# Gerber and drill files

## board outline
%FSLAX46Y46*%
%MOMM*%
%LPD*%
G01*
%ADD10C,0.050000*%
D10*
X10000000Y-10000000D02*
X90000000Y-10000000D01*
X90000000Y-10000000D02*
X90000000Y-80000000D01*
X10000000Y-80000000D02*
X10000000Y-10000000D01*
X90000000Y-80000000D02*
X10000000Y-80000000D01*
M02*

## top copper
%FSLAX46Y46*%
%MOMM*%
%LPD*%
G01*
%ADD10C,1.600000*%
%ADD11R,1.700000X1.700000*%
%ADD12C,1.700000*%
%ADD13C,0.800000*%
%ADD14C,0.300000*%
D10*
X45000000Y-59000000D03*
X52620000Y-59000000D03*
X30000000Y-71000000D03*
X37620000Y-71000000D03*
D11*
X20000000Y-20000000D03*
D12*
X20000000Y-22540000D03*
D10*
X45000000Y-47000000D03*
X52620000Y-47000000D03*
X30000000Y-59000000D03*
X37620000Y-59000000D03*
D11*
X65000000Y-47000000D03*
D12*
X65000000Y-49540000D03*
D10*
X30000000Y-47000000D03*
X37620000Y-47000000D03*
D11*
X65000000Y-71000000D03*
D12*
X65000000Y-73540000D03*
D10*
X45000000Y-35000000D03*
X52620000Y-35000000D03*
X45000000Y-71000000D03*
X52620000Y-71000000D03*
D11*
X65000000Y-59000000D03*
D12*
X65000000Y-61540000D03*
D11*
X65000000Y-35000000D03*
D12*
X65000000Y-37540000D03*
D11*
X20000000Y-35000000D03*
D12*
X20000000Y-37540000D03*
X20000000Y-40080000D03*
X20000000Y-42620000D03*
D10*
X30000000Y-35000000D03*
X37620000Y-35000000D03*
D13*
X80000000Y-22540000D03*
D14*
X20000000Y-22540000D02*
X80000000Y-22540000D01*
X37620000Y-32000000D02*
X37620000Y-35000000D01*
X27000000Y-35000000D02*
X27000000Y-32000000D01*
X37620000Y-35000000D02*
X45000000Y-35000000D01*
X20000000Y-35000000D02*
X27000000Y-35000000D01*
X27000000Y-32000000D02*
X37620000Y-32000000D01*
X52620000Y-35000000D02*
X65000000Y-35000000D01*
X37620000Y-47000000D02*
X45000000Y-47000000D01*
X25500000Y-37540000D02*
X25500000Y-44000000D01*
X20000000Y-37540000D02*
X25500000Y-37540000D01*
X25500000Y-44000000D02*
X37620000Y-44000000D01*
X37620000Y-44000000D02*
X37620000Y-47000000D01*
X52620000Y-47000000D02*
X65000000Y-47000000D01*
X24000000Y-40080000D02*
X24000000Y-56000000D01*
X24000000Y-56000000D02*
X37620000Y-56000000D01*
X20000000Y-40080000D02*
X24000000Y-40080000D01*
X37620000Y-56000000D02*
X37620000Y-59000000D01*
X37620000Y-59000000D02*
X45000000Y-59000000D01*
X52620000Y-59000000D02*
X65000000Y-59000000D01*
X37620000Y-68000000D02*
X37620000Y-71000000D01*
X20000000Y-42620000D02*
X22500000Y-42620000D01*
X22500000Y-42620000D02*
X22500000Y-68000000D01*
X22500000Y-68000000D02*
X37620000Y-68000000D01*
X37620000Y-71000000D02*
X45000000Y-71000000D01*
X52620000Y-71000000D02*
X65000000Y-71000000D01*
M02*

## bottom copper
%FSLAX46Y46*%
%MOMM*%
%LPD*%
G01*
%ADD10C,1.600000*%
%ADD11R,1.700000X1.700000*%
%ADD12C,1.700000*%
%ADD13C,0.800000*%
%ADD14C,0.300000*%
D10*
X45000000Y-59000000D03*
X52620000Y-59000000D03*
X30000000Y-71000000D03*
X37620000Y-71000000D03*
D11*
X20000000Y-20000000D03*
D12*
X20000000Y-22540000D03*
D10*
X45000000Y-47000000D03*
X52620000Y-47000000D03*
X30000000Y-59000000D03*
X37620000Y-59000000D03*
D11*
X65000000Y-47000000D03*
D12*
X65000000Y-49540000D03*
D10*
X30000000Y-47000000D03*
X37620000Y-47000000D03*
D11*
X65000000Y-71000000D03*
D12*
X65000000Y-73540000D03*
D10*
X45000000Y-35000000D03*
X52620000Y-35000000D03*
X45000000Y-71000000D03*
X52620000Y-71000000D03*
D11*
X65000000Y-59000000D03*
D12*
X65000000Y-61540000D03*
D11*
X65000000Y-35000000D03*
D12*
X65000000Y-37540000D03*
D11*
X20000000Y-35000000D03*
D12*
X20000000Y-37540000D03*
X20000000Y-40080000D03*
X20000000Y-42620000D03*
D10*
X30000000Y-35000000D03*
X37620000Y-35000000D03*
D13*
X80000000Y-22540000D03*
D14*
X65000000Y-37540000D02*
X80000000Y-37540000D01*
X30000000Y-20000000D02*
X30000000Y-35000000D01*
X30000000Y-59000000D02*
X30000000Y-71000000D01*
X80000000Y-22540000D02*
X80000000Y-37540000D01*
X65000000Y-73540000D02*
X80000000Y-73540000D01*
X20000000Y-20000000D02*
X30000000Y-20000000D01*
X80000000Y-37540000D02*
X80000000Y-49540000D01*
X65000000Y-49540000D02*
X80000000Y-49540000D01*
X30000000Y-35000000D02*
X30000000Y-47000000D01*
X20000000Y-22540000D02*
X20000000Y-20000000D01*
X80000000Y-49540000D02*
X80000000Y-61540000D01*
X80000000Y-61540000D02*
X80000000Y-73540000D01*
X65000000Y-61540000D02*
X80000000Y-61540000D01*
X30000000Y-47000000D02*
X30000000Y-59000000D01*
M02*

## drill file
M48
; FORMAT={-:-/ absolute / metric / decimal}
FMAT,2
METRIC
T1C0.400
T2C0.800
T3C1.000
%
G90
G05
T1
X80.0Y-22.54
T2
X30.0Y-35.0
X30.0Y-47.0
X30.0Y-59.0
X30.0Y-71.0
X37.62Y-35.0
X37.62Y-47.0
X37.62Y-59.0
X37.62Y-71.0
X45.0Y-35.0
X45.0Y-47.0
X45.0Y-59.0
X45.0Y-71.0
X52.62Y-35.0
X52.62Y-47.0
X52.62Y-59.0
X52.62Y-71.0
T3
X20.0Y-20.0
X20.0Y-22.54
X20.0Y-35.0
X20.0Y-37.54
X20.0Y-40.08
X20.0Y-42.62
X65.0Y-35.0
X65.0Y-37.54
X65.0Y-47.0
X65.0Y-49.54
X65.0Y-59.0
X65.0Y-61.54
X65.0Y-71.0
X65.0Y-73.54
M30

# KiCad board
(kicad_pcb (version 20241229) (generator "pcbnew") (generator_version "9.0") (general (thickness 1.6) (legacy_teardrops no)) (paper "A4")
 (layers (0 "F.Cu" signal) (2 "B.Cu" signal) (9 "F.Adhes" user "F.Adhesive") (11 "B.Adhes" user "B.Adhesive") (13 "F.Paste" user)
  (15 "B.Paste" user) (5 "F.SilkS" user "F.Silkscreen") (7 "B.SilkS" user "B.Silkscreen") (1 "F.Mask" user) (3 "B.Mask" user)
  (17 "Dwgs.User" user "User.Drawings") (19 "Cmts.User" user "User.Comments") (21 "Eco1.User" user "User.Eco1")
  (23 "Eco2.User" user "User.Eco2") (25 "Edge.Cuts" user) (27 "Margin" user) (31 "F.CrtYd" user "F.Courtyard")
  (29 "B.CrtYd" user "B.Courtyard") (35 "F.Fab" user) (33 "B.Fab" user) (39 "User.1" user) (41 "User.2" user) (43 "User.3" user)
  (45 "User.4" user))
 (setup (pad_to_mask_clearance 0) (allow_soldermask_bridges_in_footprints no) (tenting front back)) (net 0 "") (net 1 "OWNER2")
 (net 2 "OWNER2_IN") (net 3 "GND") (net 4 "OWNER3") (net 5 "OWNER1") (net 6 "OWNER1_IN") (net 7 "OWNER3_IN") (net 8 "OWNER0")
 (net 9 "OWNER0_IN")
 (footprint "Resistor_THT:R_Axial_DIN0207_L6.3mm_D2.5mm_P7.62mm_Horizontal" (layer "F.Cu") (at 45 59)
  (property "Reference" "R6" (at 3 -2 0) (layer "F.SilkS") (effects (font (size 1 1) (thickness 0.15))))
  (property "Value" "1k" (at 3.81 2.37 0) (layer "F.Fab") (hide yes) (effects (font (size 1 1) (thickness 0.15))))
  (pad "1" thru_hole circle (at 0 0) (size 1.6 1.6) (drill 0.8) (layers "*.Cu" "*.Mask") (remove_unused_layers no) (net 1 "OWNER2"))
  (pad "2" thru_hole circle (at 7.62 0) (size 1.6 1.6) (drill 0.8) (layers "*.Cu" "*.Mask") (remove_unused_layers no) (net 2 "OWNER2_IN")))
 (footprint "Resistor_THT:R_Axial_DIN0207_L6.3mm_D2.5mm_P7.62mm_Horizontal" (layer "F.Cu") (at 30 71)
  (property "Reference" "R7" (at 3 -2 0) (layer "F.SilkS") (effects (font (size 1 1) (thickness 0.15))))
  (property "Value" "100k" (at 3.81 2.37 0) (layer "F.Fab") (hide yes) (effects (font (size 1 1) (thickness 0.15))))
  (pad "1" thru_hole circle (at 0 0) (size 1.6 1.6) (drill 0.8) (layers "*.Cu" "*.Mask") (remove_unused_layers no) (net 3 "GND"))
  (pad "2" thru_hole circle (at 7.62 0) (size 1.6 1.6) (drill 0.8) (layers "*.Cu" "*.Mask") (remove_unused_layers no) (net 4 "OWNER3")))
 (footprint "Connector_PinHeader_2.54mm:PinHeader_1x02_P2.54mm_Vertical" (layer "F.Cu") (at 20 20)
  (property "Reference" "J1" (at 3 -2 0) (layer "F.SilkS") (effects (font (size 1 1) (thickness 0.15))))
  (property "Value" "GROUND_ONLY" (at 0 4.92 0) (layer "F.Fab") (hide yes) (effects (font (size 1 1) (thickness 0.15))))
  (pad "1" thru_hole rect (at 0 0) (size 1.7 1.7) (drill 1) (layers "*.Cu" "*.Mask") (remove_unused_layers no) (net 3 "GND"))
  (pad "2" thru_hole circle (at 0 2.54) (size 1.7 1.7) (drill 1) (layers "*.Cu" "*.Mask") (remove_unused_layers no) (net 3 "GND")))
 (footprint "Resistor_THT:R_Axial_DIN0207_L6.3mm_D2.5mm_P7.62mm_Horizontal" (layer "F.Cu") (at 45 47)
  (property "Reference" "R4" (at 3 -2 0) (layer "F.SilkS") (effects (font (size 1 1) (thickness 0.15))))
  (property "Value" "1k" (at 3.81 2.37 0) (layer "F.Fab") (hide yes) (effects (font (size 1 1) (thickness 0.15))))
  (pad "1" thru_hole circle (at 0 0) (size 1.6 1.6) (drill 0.8) (layers "*.Cu" "*.Mask") (remove_unused_layers no) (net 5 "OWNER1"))
  (pad "2" thru_hole circle (at 7.62 0) (size 1.6 1.6) (drill 0.8) (layers "*.Cu" "*.Mask") (remove_unused_layers no) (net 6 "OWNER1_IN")))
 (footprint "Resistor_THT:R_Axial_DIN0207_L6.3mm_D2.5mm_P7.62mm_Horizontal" (layer "F.Cu") (at 30 59)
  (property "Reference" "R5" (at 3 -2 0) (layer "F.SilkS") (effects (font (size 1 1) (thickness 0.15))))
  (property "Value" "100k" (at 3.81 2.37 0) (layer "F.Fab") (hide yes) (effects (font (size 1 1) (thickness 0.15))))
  (pad "1" thru_hole circle (at 0 0) (size 1.6 1.6) (drill 0.8) (layers "*.Cu" "*.Mask") (remove_unused_layers no) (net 3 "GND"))
  (pad "2" thru_hole circle (at 7.62 0) (size 1.6 1.6) (drill 0.8) (layers "*.Cu" "*.Mask") (remove_unused_layers no) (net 1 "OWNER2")))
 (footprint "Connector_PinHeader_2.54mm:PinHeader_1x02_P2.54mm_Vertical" (layer "F.Cu") (at 65 47)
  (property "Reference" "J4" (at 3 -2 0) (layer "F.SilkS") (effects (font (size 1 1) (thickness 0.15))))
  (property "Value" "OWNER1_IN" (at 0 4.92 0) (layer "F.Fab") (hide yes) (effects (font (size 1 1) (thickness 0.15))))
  (pad "1" thru_hole rect (at 0 0) (size 1.7 1.7) (drill 1) (layers "*.Cu" "*.Mask") (remove_unused_layers no) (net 6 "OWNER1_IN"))
  (pad "2" thru_hole circle (at 0 2.54) (size 1.7 1.7) (drill 1) (layers "*.Cu" "*.Mask") (remove_unused_layers no) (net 3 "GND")))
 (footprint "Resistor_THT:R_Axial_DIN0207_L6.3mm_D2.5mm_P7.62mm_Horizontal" (layer "F.Cu") (at 30 47)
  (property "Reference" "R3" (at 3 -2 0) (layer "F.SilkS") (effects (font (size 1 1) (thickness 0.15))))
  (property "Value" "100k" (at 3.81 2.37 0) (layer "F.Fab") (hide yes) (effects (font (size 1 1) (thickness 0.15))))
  (pad "1" thru_hole circle (at 0 0) (size 1.6 1.6) (drill 0.8) (layers "*.Cu" "*.Mask") (remove_unused_layers no) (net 3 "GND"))
  (pad "2" thru_hole circle (at 7.62 0) (size 1.6 1.6) (drill 0.8) (layers "*.Cu" "*.Mask") (remove_unused_layers no) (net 5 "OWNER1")))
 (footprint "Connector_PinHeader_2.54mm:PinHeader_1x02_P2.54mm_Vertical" (layer "F.Cu") (at 65 71)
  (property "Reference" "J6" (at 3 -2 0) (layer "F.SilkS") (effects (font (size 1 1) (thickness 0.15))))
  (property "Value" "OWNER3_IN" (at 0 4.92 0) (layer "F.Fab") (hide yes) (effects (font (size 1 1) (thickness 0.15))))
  (pad "1" thru_hole rect (at 0 0) (size 1.7 1.7) (drill 1) (layers "*.Cu" "*.Mask") (remove_unused_layers no) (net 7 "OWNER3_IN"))
  (pad "2" thru_hole circle (at 0 2.54) (size 1.7 1.7) (drill 1) (layers "*.Cu" "*.Mask") (remove_unused_layers no) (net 3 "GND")))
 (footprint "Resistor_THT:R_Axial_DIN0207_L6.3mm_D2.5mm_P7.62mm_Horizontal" (layer "F.Cu") (at 45 35)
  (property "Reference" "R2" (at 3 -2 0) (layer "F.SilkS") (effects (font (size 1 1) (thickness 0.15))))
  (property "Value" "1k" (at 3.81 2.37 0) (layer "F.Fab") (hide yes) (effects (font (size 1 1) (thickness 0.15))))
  (pad "1" thru_hole circle (at 0 0) (size 1.6 1.6) (drill 0.8) (layers "*.Cu" "*.Mask") (remove_unused_layers no) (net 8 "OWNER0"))
  (pad "2" thru_hole circle (at 7.62 0) (size 1.6 1.6) (drill 0.8) (layers "*.Cu" "*.Mask") (remove_unused_layers no) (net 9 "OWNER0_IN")))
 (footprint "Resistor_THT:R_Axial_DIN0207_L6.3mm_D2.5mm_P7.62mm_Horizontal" (layer "F.Cu") (at 45 71)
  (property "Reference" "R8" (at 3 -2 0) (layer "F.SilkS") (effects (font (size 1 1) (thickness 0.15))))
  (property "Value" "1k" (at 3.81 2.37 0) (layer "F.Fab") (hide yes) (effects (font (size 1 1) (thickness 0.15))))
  (pad "1" thru_hole circle (at 0 0) (size 1.6 1.6) (drill 0.8) (layers "*.Cu" "*.Mask") (remove_unused_layers no) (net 4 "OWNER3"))
  (pad "2" thru_hole circle (at 7.62 0) (size 1.6 1.6) (drill 0.8) (layers "*.Cu" "*.Mask") (remove_unused_layers no) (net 7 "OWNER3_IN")))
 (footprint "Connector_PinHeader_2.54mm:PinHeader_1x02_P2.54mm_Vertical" (layer "F.Cu") (at 65 59)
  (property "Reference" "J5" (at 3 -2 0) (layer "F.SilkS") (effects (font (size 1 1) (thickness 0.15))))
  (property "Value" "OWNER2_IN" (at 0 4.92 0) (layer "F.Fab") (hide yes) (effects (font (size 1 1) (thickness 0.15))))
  (pad "1" thru_hole rect (at 0 0) (size 1.7 1.7) (drill 1) (layers "*.Cu" "*.Mask") (remove_unused_layers no) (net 2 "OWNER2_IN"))
  (pad "2" thru_hole circle (at 0 2.54) (size 1.7 1.7) (drill 1) (layers "*.Cu" "*.Mask") (remove_unused_layers no) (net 3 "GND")))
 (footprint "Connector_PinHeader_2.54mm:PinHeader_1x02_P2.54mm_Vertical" (layer "F.Cu") (at 65 35)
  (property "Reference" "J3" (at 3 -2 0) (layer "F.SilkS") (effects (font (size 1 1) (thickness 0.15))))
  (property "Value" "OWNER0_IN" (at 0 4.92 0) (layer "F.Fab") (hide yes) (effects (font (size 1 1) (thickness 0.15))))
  (pad "1" thru_hole rect (at 0 0) (size 1.7 1.7) (drill 1) (layers "*.Cu" "*.Mask") (remove_unused_layers no) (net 9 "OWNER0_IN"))
  (pad "2" thru_hole circle (at 0 2.54) (size 1.7 1.7) (drill 1) (layers "*.Cu" "*.Mask") (remove_unused_layers no) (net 3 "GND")))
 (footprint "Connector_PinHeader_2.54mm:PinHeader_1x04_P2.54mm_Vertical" (layer "F.Cu") (at 20 35)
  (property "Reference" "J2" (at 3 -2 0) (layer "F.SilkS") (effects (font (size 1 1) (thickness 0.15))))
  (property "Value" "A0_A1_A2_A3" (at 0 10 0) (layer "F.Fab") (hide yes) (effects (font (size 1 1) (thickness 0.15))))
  (pad "1" thru_hole rect (at 0 0) (size 1.7 1.7) (drill 1) (layers "*.Cu" "*.Mask") (remove_unused_layers no) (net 8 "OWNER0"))
  (pad "2" thru_hole circle (at 0 2.54) (size 1.7 1.7) (drill 1) (layers "*.Cu" "*.Mask") (remove_unused_layers no) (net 5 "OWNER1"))
  (pad "3" thru_hole circle (at 0 5.08) (size 1.7 1.7) (drill 1) (layers "*.Cu" "*.Mask") (remove_unused_layers no) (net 1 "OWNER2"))
  (pad "4" thru_hole circle (at 0 7.62) (size 1.7 1.7) (drill 1) (layers "*.Cu" "*.Mask") (remove_unused_layers no) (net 4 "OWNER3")))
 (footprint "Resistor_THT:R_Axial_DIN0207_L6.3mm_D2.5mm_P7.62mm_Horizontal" (layer "F.Cu") (at 30 35)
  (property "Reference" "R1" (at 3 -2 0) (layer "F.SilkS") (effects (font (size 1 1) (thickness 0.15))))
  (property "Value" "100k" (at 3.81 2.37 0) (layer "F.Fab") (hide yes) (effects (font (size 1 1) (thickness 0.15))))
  (pad "1" thru_hole circle (at 0 0) (size 1.6 1.6) (drill 0.8) (layers "*.Cu" "*.Mask") (remove_unused_layers no) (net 3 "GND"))
  (pad "2" thru_hole circle (at 7.62 0) (size 1.6 1.6) (drill 0.8) (layers "*.Cu" "*.Mask") (remove_unused_layers no) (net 8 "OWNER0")))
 (gr_line (start 10 10) (end 90 10) (stroke (width 0.05) (type default)) (layer "Edge.Cuts"))
 (gr_line (start 90 10) (end 90 80) (stroke (width 0.05) (type default)) (layer "Edge.Cuts"))
 (gr_line (start 10 80) (end 10 10) (stroke (width 0.05) (type default)) (layer "Edge.Cuts"))
 (gr_line (start 90 80) (end 10 80) (stroke (width 0.05) (type default)) (layer "Edge.Cuts"))
 (segment (start 20 22.54) (end 80 22.54) (width 0.3) (layer "F.Cu") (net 3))
 (via (at 80 22.54) (size 0.8) (drill 0.4) (layers "F.Cu" "B.Cu") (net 3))
 (segment (start 65 37.54) (end 80 37.54) (width 0.3) (layer "B.Cu") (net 3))
 (segment (start 30 20) (end 30 35) (width 0.3) (layer "B.Cu") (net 3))
 (segment (start 30 59) (end 30 71) (width 0.3) (layer "B.Cu") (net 3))
 (segment (start 80 22.54) (end 80 37.54) (width 0.3) (layer "B.Cu") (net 3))
 (segment (start 65 73.54) (end 80 73.54) (width 0.3) (layer "B.Cu") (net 3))
 (segment (start 20 20) (end 30 20) (width 0.3) (layer "B.Cu") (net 3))
 (segment (start 80 37.54) (end 80 49.54) (width 0.3) (layer "B.Cu") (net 3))
 (segment (start 65 49.54) (end 80 49.54) (width 0.3) (layer "B.Cu") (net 3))
 (segment (start 30 35) (end 30 47) (width 0.3) (layer "B.Cu") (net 3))
 (segment (start 20 22.54) (end 20 20) (width 0.3) (layer "B.Cu") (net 3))
 (segment (start 80 49.54) (end 80 61.54) (width 0.3) (layer "B.Cu") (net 3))
 (segment (start 80 61.54) (end 80 73.54) (width 0.3) (layer "B.Cu") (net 3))
 (segment (start 65 61.54) (end 80 61.54) (width 0.3) (layer "B.Cu") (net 3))
 (segment (start 30 47) (end 30 59) (width 0.3) (layer "B.Cu") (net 3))
 (segment (start 37.62 32) (end 37.62 35) (width 0.3) (layer "F.Cu") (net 8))
 (segment (start 27 35) (end 27 32) (width 0.3) (layer "F.Cu") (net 8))
 (segment (start 37.62 35) (end 45 35) (width 0.3) (layer "F.Cu") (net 8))
 (segment (start 20 35) (end 27 35) (width 0.3) (layer "F.Cu") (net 8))
 (segment (start 27 32) (end 37.62 32) (width 0.3) (layer "F.Cu") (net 8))
 (segment (start 52.62 35) (end 65 35) (width 0.3) (layer "F.Cu") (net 9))
 (segment (start 37.62 47) (end 45 47) (width 0.3) (layer "F.Cu") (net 5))
 (segment (start 25.5 37.54) (end 25.5 44) (width 0.3) (layer "F.Cu") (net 5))
 (segment (start 20 37.54) (end 25.5 37.54) (width 0.3) (layer "F.Cu") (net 5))
 (segment (start 25.5 44) (end 37.62 44) (width 0.3) (layer "F.Cu") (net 5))
 (segment (start 37.62 44) (end 37.62 47) (width 0.3) (layer "F.Cu") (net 5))
 (segment (start 52.62 47) (end 65 47) (width 0.3) (layer "F.Cu") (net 6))
 (segment (start 24 40.08) (end 24 56) (width 0.3) (layer "F.Cu") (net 1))
 (segment (start 24 56) (end 37.62 56) (width 0.3) (layer "F.Cu") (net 1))
 (segment (start 20 40.08) (end 24 40.08) (width 0.3) (layer "F.Cu") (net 1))
 (segment (start 37.62 56) (end 37.62 59) (width 0.3) (layer "F.Cu") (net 1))
 (segment (start 37.62 59) (end 45 59) (width 0.3) (layer "F.Cu") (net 1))
 (segment (start 52.62 59) (end 65 59) (width 0.3) (layer "F.Cu") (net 2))
 (segment (start 37.62 68) (end 37.62 71) (width 0.3) (layer "F.Cu") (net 4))
 (segment (start 20 42.62) (end 22.5 42.62) (width 0.3) (layer "F.Cu") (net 4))
 (segment (start 22.5 42.62) (end 22.5 68) (width 0.3) (layer "F.Cu") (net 4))
 (segment (start 22.5 68) (end 37.62 68) (width 0.3) (layer "F.Cu") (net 4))
 (segment (start 37.62 71) (end 45 71) (width 0.3) (layer "F.Cu") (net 4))
 (segment (start 52.62 71) (end 65 71) (width 0.3) (layer "F.Cu") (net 7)))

